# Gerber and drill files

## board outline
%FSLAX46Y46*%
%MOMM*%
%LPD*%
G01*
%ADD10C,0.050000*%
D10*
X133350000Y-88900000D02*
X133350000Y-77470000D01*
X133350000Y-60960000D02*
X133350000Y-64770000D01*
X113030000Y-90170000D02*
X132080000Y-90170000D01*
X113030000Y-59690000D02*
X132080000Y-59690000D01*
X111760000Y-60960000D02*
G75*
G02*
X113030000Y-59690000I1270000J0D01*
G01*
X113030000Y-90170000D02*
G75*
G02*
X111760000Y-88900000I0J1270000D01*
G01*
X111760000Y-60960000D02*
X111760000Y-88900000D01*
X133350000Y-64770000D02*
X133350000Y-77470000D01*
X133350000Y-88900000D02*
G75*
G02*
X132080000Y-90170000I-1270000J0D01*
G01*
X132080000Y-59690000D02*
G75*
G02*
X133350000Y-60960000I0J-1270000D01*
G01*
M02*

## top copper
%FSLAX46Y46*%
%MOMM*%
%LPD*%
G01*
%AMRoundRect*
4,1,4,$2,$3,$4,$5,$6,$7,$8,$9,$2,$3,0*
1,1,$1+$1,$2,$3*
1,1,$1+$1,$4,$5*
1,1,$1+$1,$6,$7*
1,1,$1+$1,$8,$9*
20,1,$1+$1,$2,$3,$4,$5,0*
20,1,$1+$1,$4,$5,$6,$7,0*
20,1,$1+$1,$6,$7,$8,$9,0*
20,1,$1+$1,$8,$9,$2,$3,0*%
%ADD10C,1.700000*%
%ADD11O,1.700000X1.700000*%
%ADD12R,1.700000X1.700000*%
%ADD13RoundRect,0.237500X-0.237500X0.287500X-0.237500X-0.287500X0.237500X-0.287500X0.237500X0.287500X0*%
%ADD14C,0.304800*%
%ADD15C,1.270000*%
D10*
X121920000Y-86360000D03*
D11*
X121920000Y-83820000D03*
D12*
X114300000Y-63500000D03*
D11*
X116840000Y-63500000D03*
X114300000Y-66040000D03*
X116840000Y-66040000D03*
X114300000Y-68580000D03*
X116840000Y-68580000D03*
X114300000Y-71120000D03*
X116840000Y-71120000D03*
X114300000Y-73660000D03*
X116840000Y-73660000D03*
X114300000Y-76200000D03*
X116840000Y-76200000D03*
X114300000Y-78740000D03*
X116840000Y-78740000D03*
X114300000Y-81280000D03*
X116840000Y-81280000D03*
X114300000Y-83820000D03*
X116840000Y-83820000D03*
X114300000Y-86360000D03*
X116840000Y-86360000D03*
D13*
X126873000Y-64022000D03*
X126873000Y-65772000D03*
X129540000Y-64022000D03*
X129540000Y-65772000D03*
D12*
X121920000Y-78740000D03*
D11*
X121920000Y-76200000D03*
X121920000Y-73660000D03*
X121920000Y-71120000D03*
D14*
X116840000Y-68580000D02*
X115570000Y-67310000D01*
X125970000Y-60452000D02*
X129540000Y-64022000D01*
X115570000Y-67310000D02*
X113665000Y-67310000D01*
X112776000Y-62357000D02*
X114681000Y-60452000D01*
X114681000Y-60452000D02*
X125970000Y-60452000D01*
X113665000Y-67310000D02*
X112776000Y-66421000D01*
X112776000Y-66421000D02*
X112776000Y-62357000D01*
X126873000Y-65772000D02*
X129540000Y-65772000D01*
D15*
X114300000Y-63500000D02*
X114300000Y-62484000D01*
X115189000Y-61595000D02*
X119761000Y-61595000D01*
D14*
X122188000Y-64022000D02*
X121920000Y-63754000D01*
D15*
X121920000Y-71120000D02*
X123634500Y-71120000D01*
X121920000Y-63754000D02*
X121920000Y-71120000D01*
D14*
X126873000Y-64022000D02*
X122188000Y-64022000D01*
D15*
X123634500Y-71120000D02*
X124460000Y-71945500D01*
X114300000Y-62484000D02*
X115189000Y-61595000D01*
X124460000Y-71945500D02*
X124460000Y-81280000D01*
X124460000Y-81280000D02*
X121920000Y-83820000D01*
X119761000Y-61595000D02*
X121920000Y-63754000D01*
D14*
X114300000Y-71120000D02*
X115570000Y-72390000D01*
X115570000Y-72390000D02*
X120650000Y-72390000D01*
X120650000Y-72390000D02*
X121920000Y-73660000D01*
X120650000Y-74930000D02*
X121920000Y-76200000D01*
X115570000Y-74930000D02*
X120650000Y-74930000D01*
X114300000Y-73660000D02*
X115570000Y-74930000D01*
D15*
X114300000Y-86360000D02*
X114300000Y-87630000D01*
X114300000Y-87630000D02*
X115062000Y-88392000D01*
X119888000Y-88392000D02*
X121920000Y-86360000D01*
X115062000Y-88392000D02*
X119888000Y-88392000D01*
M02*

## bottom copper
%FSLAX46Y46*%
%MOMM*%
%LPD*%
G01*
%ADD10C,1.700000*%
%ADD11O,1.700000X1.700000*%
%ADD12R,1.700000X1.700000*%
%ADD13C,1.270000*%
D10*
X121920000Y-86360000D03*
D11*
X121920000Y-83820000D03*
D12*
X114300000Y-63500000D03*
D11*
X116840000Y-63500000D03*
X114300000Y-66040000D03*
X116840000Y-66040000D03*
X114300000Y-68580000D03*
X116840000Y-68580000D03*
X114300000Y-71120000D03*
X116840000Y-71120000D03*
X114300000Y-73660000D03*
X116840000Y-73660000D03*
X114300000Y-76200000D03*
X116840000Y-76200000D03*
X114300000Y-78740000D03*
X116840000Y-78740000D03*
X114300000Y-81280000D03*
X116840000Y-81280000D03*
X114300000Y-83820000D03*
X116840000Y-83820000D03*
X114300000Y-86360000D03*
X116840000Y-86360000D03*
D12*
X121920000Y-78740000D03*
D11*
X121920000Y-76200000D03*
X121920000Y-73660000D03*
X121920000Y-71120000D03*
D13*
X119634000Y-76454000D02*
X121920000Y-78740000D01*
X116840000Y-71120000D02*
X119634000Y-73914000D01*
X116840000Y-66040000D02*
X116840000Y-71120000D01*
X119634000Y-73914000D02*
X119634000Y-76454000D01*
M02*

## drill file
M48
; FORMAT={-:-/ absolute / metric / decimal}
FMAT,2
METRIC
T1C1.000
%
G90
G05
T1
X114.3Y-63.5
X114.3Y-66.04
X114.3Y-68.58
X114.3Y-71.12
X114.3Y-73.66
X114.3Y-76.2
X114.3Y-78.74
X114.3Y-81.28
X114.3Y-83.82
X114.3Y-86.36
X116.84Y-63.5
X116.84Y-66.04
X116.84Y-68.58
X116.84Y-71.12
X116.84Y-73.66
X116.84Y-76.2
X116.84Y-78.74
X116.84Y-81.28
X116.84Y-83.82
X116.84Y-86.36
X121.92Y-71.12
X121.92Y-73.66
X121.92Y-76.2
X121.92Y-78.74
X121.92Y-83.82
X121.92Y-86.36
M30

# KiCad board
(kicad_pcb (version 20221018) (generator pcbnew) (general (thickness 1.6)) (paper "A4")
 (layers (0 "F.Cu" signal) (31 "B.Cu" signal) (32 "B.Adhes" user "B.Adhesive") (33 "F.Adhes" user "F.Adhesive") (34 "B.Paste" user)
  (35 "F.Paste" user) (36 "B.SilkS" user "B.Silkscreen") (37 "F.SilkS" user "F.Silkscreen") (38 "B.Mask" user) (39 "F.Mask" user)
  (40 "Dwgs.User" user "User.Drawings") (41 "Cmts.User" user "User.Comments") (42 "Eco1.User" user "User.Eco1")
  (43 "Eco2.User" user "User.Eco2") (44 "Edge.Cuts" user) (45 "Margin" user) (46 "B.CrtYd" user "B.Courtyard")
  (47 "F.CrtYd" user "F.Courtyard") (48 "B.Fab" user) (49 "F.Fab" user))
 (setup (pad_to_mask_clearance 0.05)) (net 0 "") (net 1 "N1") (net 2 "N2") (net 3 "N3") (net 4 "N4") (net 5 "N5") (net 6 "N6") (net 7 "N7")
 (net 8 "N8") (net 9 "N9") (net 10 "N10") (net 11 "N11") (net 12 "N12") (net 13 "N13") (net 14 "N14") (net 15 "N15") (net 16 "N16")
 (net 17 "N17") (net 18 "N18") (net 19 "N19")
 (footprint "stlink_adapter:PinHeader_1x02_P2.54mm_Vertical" (layer "F.Cu") (at 121.92 86.36 180)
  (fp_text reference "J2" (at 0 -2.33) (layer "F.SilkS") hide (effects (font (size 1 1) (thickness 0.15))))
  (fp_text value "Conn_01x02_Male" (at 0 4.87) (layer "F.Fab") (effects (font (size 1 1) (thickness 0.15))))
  (pad "1" thru_hole circle (at 0 0 180) (size 1.7 1.7) (drill 1) (layers "*.Cu" "*.Mask") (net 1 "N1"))
  (pad "2" thru_hole oval (at 0 2.54 180) (size 1.7 1.7) (drill 1) (layers "*.Cu" "*.Mask") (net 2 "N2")))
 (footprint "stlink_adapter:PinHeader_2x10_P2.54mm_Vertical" (layer "F.Cu") (at 114.3 63.5)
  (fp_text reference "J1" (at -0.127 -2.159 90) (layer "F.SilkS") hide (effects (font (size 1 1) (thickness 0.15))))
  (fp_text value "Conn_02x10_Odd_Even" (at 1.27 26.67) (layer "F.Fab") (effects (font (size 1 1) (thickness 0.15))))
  (pad "1" thru_hole rect (at 0 0) (size 1.7 1.7) (drill 1) (layers "*.Cu" "*.Mask") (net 2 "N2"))
  (pad "2" thru_hole oval (at 2.54 0) (size 1.7 1.7) (drill 1) (layers "*.Cu" "*.Mask") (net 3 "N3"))
  (pad "3" thru_hole oval (at 0 2.54) (size 1.7 1.7) (drill 1) (layers "*.Cu" "*.Mask") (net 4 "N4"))
  (pad "4" thru_hole oval (at 2.54 2.54) (size 1.7 1.7) (drill 1) (layers "*.Cu" "*.Mask") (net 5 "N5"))
  (pad "5" thru_hole oval (at 0 5.08) (size 1.7 1.7) (drill 1) (layers "*.Cu" "*.Mask") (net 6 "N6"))
  (pad "6" thru_hole oval (at 2.54 5.08) (size 1.7 1.7) (drill 1) (layers "*.Cu" "*.Mask") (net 5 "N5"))
  (pad "7" thru_hole oval (at 0 7.62) (size 1.7 1.7) (drill 1) (layers "*.Cu" "*.Mask") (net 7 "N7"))
  (pad "8" thru_hole oval (at 2.54 7.62) (size 1.7 1.7) (drill 1) (layers "*.Cu" "*.Mask") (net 5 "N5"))
  (pad "9" thru_hole oval (at 0 10.16) (size 1.7 1.7) (drill 1) (layers "*.Cu" "*.Mask") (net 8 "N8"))
  (pad "10" thru_hole oval (at 2.54 10.16) (size 1.7 1.7) (drill 1) (layers "*.Cu" "*.Mask") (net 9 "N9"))
  (pad "11" thru_hole oval (at 0 12.7) (size 1.7 1.7) (drill 1) (layers "*.Cu" "*.Mask") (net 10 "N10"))
  (pad "12" thru_hole oval (at 2.54 12.7) (size 1.7 1.7) (drill 1) (layers "*.Cu" "*.Mask") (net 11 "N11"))
  (pad "13" thru_hole oval (at 0 15.24) (size 1.7 1.7) (drill 1) (layers "*.Cu" "*.Mask") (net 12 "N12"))
  (pad "14" thru_hole oval (at 2.54 15.24) (size 1.7 1.7) (drill 1) (layers "*.Cu" "*.Mask") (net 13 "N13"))
  (pad "15" thru_hole oval (at 0 17.78) (size 1.7 1.7) (drill 1) (layers "*.Cu" "*.Mask") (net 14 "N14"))
  (pad "16" thru_hole oval (at 2.54 17.78) (size 1.7 1.7) (drill 1) (layers "*.Cu" "*.Mask") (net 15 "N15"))
  (pad "17" thru_hole oval (at 0 20.32) (size 1.7 1.7) (drill 1) (layers "*.Cu" "*.Mask") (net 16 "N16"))
  (pad "18" thru_hole oval (at 2.54 20.32) (size 1.7 1.7) (drill 1) (layers "*.Cu" "*.Mask") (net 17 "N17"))
  (pad "19" thru_hole oval (at 0 22.86) (size 1.7 1.7) (drill 1) (layers "*.Cu" "*.Mask") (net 1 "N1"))
  (pad "20" thru_hole oval (at 2.54 22.86) (size 1.7 1.7) (drill 1) (layers "*.Cu" "*.Mask") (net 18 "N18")))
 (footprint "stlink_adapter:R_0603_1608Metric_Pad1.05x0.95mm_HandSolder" (layer "F.Cu") (at 126.873 64.897 -90)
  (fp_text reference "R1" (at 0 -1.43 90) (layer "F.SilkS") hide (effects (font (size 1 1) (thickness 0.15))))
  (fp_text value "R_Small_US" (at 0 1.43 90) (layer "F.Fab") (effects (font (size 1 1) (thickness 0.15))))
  (pad "1" smd roundrect (at -0.875 0 270) (size 1.05 0.95) (layers "F.Cu" "F.Paste" "F.Mask") (roundrect_rratio 0.25) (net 2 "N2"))
  (pad "2" smd roundrect (at 0.875 0 270) (size 1.05 0.95) (layers "F.Cu" "F.Paste" "F.Mask") (roundrect_rratio 0.25) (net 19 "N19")))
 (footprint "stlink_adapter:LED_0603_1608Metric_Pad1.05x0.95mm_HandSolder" (layer "F.Cu") (at 129.54 64.897 -90)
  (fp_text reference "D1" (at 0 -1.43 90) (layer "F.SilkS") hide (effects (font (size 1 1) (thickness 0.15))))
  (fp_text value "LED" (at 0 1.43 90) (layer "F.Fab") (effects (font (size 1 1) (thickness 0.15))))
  (pad "1" smd roundrect (at -0.875 0 270) (size 1.05 0.95) (layers "F.Cu" "F.Paste" "F.Mask") (roundrect_rratio 0.25) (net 5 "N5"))
  (pad "2" smd roundrect (at 0.875 0 270) (size 1.05 0.95) (layers "F.Cu" "F.Paste" "F.Mask") (roundrect_rratio 0.25) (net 19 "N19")))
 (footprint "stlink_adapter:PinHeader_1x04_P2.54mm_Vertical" (layer "F.Cu") (at 121.92 78.74 180)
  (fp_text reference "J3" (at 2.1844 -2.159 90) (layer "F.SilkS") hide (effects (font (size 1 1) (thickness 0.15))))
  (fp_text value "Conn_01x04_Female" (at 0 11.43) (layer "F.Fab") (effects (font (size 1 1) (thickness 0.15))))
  (pad "1" thru_hole rect (at 0 0 180) (size 1.7 1.7) (drill 1) (layers "*.Cu" "*.Mask") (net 5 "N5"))
  (pad "2" thru_hole oval (at 0 2.54 180) (size 1.7 1.7) (drill 1) (layers "*.Cu" "*.Mask") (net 8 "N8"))
  (pad "3" thru_hole oval (at 0 5.08 180) (size 1.7 1.7) (drill 1) (layers "*.Cu" "*.Mask") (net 7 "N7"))
  (pad "4" thru_hole oval (at 0 7.62 180) (size 1.7 1.7) (drill 1) (layers "*.Cu" "*.Mask") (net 2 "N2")))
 (gr_line (start 133.35 88.9) (end 133.35 77.47) (stroke (width 0.05) (type solid)) (layer "Edge.Cuts"))
 (gr_line (start 133.35 60.96) (end 133.35 64.77) (stroke (width 0.05) (type solid)) (layer "Edge.Cuts"))
 (gr_line (start 113.03 90.17) (end 132.08 90.17) (stroke (width 0.05) (type solid)) (layer "Edge.Cuts"))
 (gr_line (start 113.03 59.69) (end 132.08 59.69) (stroke (width 0.05) (type solid)) (layer "Edge.Cuts"))
 (gr_arc (start 111.76 60.96) (mid 112.131974 60.061974) (end 113.03 59.69) (stroke (width 0.05) (type solid)) (layer "Edge.Cuts"))
 (gr_arc (start 113.03 90.17) (mid 112.131974 89.798026) (end 111.76 88.9) (stroke (width 0.05) (type solid)) (layer "Edge.Cuts"))
 (gr_line (start 111.76 60.96) (end 111.76 88.9) (stroke (width 0.05) (type solid)) (layer "Edge.Cuts"))
 (gr_line (start 133.35 64.77) (end 133.35 77.47) (stroke (width 0.05) (type solid)) (layer "Edge.Cuts"))
 (gr_arc (start 133.35 88.9) (mid 132.978026 89.798026) (end 132.08 90.17) (stroke (width 0.05) (type solid)) (layer "Edge.Cuts"))
 (gr_arc (start 132.08 59.69) (mid 132.978026 60.061974) (end 133.35 60.96) (stroke (width 0.05) (type solid)) (layer "Edge.Cuts"))
 (segment (start 116.84 68.58) (end 115.57 67.31) (width 0.3048) (layer "F.Cu") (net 5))
 (segment (start 125.97 60.452) (end 129.54 64.022) (width 0.3048) (layer "F.Cu") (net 5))
 (segment (start 115.57 67.31) (end 113.665 67.31) (width 0.3048) (layer "F.Cu") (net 5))
 (segment (start 112.776 62.357) (end 114.681 60.452) (width 0.3048) (layer "F.Cu") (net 5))
 (segment (start 114.681 60.452) (end 125.97 60.452) (width 0.3048) (layer "F.Cu") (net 5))
 (segment (start 113.665 67.31) (end 112.776 66.421) (width 0.3048) (layer "F.Cu") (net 5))
 (segment (start 112.776 66.421) (end 112.776 62.357) (width 0.3048) (layer "F.Cu") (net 5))
 (segment (start 119.634 76.454) (end 121.92 78.74) (width 1.27) (layer "B.Cu") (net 5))
 (segment (start 116.84 71.12) (end 119.634 73.914) (width 1.27) (layer "B.Cu") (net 5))
 (segment (start 116.84 66.04) (end 116.84 71.12) (width 1.27) (layer "B.Cu") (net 5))
 (segment (start 119.634 73.914) (end 119.634 76.454) (width 1.27) (layer "B.Cu") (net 5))
 (segment (start 126.873 65.772) (end 129.54 65.772) (width 0.3048) (layer "F.Cu") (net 19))
 (segment (start 114.3 63.5) (end 114.3 62.484) (width 1.27) (layer "F.Cu") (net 2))
 (segment (start 115.189 61.595) (end 119.761 61.595) (width 1.27) (layer "F.Cu") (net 2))
 (segment (start 122.188 64.022) (end 121.92 63.754) (width 0.3048) (layer "F.Cu") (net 2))
 (segment (start 121.92 71.12) (end 123.6345 71.12) (width 1.27) (layer "F.Cu") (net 2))
 (segment (start 121.92 63.754) (end 121.92 71.12) (width 1.27) (layer "F.Cu") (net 2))
 (segment (start 126.873 64.022) (end 122.188 64.022) (width 0.3048) (layer "F.Cu") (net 2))
 (segment (start 123.6345 71.12) (end 124.46 71.9455) (width 1.27) (layer "F.Cu") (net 2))
 (segment (start 114.3 62.484) (end 115.189 61.595) (width 1.27) (layer "F.Cu") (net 2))
 (segment (start 124.46 71.9455) (end 124.46 81.28) (width 1.27) (layer "F.Cu") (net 2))
 (segment (start 124.46 81.28) (end 121.92 83.82) (width 1.27) (layer "F.Cu") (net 2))
 (segment (start 119.761 61.595) (end 121.92 63.754) (width 1.27) (layer "F.Cu") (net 2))
 (segment (start 114.3 71.12) (end 115.57 72.39) (width 0.3048) (layer "F.Cu") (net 7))
 (segment (start 115.57 72.39) (end 120.65 72.39) (width 0.3048) (layer "F.Cu") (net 7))
 (segment (start 120.65 72.39) (end 121.92 73.66) (width 0.3048) (layer "F.Cu") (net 7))
 (segment (start 120.65 74.93) (end 121.92 76.2) (width 0.3048) (layer "F.Cu") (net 8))
 (segment (start 115.57 74.93) (end 120.65 74.93) (width 0.3048) (layer "F.Cu") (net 8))
 (segment (start 114.3 73.66) (end 115.57 74.93) (width 0.3048) (layer "F.Cu") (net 8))
 (segment (start 114.3 86.36) (end 114.3 87.63) (width 1.27) (layer "F.Cu") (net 1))
 (segment (start 114.3 87.63) (end 115.062 88.392) (width 1.27) (layer "F.Cu") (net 1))
 (segment (start 119.888 88.392) (end 121.92 86.36) (width 1.27) (layer "F.Cu") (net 1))
 (segment (start 115.062 88.392) (end 119.888 88.392) (width 1.27) (layer "F.Cu") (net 1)))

